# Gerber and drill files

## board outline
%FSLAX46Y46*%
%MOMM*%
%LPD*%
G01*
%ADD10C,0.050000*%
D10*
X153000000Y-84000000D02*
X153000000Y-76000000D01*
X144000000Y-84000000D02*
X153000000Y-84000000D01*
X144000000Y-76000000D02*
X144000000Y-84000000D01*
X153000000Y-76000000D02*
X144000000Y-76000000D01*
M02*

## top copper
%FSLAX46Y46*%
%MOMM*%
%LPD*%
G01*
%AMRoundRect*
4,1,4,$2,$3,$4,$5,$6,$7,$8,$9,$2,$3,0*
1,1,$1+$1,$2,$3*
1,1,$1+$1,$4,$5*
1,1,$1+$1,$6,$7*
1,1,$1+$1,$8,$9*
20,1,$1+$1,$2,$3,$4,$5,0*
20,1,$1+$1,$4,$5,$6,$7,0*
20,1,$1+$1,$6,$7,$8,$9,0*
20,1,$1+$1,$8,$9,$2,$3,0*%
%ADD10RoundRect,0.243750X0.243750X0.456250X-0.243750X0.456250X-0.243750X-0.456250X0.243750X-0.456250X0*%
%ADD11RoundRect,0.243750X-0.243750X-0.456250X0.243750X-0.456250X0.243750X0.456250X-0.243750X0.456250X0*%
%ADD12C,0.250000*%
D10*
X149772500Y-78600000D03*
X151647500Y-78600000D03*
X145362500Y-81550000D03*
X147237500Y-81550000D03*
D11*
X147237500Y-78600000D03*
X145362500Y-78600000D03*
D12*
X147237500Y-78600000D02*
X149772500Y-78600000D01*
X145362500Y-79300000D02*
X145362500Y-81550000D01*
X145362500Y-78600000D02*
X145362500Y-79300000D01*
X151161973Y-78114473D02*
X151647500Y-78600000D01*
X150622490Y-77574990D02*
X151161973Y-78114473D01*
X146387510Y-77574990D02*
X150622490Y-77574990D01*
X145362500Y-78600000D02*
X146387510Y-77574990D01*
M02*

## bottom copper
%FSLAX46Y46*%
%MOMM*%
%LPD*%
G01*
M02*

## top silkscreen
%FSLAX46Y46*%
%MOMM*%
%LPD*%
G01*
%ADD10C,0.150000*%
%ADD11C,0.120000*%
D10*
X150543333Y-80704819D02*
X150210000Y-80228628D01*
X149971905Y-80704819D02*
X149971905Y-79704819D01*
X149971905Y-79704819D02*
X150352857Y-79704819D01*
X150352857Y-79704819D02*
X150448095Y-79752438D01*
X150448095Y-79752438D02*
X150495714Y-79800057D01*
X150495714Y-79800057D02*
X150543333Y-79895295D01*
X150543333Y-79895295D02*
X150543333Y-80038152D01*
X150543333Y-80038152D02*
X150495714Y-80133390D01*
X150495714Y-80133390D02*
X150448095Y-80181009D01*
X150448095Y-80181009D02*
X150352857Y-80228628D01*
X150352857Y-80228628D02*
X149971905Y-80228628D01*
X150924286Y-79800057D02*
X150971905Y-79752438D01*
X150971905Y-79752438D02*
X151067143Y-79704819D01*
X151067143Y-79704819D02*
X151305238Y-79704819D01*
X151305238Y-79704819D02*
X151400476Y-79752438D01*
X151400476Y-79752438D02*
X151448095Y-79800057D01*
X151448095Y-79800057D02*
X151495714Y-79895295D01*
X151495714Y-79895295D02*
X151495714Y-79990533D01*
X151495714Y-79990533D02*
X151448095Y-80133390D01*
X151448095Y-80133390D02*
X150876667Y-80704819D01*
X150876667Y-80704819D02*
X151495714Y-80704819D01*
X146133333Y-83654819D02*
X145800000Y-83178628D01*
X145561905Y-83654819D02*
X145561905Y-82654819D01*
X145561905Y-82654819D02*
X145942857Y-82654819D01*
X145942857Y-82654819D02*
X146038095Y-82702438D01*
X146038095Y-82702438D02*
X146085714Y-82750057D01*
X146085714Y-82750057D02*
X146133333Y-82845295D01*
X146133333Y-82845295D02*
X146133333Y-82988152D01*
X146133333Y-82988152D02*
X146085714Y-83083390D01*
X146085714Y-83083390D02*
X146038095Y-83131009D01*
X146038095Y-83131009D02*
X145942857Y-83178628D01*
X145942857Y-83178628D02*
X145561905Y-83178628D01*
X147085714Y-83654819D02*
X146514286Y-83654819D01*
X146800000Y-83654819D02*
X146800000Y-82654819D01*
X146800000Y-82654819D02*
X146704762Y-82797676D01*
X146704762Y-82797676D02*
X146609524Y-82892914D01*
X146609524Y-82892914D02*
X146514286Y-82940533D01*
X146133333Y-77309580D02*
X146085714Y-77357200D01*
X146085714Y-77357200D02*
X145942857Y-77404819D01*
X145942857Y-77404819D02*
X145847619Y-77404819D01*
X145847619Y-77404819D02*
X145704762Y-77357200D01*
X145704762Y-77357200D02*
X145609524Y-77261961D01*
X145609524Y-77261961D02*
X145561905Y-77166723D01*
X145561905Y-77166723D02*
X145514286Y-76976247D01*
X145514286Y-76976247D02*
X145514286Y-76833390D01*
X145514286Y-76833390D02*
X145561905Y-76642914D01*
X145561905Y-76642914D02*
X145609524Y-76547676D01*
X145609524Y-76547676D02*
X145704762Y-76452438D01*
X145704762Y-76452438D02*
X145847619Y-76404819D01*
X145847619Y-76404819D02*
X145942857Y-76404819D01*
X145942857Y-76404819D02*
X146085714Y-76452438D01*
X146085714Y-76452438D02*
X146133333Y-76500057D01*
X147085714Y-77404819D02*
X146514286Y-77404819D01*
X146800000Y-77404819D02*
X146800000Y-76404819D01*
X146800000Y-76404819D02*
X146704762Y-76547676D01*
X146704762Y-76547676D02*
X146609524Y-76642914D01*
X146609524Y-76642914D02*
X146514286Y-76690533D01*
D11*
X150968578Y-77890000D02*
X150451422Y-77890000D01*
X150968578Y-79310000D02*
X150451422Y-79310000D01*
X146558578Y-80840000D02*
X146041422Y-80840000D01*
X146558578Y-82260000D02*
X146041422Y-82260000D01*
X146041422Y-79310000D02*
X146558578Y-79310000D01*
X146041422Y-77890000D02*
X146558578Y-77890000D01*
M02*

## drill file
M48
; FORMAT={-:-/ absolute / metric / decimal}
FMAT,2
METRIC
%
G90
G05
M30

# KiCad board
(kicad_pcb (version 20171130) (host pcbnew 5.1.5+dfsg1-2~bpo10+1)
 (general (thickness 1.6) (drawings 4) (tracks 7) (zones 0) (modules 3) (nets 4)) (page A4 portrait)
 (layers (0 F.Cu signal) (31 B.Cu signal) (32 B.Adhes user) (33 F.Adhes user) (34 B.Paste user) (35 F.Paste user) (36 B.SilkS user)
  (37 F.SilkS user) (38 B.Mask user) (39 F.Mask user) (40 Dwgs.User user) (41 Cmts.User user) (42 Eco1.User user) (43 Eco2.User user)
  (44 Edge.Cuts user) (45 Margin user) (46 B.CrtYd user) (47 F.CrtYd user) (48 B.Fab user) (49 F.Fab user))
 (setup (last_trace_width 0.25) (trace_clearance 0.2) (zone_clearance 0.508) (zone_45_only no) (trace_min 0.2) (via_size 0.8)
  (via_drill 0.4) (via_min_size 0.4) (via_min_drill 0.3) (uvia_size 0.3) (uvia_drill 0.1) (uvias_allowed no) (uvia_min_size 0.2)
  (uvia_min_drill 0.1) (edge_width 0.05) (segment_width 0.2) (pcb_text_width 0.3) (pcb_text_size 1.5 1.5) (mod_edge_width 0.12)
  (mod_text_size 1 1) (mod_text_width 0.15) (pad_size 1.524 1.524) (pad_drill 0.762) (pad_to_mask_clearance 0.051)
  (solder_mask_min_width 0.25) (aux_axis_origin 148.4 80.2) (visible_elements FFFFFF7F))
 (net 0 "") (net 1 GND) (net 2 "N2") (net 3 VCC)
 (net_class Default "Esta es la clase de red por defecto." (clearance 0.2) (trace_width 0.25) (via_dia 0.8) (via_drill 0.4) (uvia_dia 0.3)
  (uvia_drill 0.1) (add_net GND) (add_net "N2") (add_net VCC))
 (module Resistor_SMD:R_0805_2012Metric (layer F.Cu) (at 150.71 78.6 180)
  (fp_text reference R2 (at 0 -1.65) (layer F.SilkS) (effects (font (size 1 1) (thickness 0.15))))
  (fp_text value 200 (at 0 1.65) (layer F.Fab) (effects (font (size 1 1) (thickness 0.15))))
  (fp_line (start -0.258578 0.71) (end 0.258578 0.71) (layer F.SilkS) (width 0.12))
  (fp_line (start -0.258578 -0.71) (end 0.258578 -0.71) (layer F.SilkS) (width 0.12))
  (pad 2 smd roundrect (at 0.9375 0 180) (size 0.975 1.4) (layers F.Cu F.Paste F.Mask) (roundrect_rratio 0.25) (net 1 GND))
  (pad 1 smd roundrect (at -0.9375 0 180) (size 0.975 1.4) (layers F.Cu F.Paste F.Mask) (roundrect_rratio 0.25) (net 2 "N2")))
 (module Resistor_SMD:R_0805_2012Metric (layer F.Cu) (at 146.3 81.55 180)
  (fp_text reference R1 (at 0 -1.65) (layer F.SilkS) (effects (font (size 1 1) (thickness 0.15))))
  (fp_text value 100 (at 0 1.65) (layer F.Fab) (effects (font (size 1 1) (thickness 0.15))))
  (fp_line (start -0.258578 0.71) (end 0.258578 0.71) (layer F.SilkS) (width 0.12))
  (fp_line (start -0.258578 -0.71) (end 0.258578 -0.71) (layer F.SilkS) (width 0.12))
  (pad 2 smd roundrect (at 0.9375 0 180) (size 0.975 1.4) (layers F.Cu F.Paste F.Mask) (roundrect_rratio 0.25) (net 2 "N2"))
  (pad 1 smd roundrect (at -0.9375 0 180) (size 0.975 1.4) (layers F.Cu F.Paste F.Mask) (roundrect_rratio 0.25) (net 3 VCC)))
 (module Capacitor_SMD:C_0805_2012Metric (layer F.Cu) (at 146.3 78.6)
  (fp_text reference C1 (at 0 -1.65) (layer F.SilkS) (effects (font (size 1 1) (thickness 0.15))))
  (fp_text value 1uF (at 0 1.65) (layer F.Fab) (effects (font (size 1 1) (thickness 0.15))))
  (fp_line (start -0.258578 0.71) (end 0.258578 0.71) (layer F.SilkS) (width 0.12))
  (fp_line (start -0.258578 -0.71) (end 0.258578 -0.71) (layer F.SilkS) (width 0.12))
  (pad 2 smd roundrect (at 0.9375 0) (size 0.975 1.4) (layers F.Cu F.Paste F.Mask) (roundrect_rratio 0.25) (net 1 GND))
  (pad 1 smd roundrect (at -0.9375 0) (size 0.975 1.4) (layers F.Cu F.Paste F.Mask) (roundrect_rratio 0.25) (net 2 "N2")))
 (gr_line (start 153 84) (end 153 76) (layer Edge.Cuts) (width 0.05))
 (gr_line (start 144 84) (end 153 84) (layer Edge.Cuts) (width 0.05))
 (gr_line (start 144 76) (end 144 84) (layer Edge.Cuts) (width 0.05))
 (gr_line (start 153 76) (end 144 76) (layer Edge.Cuts) (width 0.05))
 (segment (start 147.2375 78.6) (end 149.7725 78.6) (width 0.25) (layer F.Cu) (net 1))
 (segment (start 145.3625 79.3) (end 145.3625 81.55) (width 0.25) (layer F.Cu) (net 2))
 (segment (start 145.3625 78.6) (end 145.3625 79.3) (width 0.25) (layer F.Cu) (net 2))
 (segment (start 151.161973 78.114473) (end 151.6475 78.6) (width 0.25) (layer F.Cu) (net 2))
 (segment (start 150.62249 77.57499) (end 151.161973 78.114473) (width 0.25) (layer F.Cu) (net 2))
 (segment (start 146.38751 77.57499) (end 150.62249 77.57499) (width 0.25) (layer F.Cu) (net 2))
 (segment (start 145.3625 78.6) (end 146.38751 77.57499) (width 0.25) (layer F.Cu) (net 2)))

